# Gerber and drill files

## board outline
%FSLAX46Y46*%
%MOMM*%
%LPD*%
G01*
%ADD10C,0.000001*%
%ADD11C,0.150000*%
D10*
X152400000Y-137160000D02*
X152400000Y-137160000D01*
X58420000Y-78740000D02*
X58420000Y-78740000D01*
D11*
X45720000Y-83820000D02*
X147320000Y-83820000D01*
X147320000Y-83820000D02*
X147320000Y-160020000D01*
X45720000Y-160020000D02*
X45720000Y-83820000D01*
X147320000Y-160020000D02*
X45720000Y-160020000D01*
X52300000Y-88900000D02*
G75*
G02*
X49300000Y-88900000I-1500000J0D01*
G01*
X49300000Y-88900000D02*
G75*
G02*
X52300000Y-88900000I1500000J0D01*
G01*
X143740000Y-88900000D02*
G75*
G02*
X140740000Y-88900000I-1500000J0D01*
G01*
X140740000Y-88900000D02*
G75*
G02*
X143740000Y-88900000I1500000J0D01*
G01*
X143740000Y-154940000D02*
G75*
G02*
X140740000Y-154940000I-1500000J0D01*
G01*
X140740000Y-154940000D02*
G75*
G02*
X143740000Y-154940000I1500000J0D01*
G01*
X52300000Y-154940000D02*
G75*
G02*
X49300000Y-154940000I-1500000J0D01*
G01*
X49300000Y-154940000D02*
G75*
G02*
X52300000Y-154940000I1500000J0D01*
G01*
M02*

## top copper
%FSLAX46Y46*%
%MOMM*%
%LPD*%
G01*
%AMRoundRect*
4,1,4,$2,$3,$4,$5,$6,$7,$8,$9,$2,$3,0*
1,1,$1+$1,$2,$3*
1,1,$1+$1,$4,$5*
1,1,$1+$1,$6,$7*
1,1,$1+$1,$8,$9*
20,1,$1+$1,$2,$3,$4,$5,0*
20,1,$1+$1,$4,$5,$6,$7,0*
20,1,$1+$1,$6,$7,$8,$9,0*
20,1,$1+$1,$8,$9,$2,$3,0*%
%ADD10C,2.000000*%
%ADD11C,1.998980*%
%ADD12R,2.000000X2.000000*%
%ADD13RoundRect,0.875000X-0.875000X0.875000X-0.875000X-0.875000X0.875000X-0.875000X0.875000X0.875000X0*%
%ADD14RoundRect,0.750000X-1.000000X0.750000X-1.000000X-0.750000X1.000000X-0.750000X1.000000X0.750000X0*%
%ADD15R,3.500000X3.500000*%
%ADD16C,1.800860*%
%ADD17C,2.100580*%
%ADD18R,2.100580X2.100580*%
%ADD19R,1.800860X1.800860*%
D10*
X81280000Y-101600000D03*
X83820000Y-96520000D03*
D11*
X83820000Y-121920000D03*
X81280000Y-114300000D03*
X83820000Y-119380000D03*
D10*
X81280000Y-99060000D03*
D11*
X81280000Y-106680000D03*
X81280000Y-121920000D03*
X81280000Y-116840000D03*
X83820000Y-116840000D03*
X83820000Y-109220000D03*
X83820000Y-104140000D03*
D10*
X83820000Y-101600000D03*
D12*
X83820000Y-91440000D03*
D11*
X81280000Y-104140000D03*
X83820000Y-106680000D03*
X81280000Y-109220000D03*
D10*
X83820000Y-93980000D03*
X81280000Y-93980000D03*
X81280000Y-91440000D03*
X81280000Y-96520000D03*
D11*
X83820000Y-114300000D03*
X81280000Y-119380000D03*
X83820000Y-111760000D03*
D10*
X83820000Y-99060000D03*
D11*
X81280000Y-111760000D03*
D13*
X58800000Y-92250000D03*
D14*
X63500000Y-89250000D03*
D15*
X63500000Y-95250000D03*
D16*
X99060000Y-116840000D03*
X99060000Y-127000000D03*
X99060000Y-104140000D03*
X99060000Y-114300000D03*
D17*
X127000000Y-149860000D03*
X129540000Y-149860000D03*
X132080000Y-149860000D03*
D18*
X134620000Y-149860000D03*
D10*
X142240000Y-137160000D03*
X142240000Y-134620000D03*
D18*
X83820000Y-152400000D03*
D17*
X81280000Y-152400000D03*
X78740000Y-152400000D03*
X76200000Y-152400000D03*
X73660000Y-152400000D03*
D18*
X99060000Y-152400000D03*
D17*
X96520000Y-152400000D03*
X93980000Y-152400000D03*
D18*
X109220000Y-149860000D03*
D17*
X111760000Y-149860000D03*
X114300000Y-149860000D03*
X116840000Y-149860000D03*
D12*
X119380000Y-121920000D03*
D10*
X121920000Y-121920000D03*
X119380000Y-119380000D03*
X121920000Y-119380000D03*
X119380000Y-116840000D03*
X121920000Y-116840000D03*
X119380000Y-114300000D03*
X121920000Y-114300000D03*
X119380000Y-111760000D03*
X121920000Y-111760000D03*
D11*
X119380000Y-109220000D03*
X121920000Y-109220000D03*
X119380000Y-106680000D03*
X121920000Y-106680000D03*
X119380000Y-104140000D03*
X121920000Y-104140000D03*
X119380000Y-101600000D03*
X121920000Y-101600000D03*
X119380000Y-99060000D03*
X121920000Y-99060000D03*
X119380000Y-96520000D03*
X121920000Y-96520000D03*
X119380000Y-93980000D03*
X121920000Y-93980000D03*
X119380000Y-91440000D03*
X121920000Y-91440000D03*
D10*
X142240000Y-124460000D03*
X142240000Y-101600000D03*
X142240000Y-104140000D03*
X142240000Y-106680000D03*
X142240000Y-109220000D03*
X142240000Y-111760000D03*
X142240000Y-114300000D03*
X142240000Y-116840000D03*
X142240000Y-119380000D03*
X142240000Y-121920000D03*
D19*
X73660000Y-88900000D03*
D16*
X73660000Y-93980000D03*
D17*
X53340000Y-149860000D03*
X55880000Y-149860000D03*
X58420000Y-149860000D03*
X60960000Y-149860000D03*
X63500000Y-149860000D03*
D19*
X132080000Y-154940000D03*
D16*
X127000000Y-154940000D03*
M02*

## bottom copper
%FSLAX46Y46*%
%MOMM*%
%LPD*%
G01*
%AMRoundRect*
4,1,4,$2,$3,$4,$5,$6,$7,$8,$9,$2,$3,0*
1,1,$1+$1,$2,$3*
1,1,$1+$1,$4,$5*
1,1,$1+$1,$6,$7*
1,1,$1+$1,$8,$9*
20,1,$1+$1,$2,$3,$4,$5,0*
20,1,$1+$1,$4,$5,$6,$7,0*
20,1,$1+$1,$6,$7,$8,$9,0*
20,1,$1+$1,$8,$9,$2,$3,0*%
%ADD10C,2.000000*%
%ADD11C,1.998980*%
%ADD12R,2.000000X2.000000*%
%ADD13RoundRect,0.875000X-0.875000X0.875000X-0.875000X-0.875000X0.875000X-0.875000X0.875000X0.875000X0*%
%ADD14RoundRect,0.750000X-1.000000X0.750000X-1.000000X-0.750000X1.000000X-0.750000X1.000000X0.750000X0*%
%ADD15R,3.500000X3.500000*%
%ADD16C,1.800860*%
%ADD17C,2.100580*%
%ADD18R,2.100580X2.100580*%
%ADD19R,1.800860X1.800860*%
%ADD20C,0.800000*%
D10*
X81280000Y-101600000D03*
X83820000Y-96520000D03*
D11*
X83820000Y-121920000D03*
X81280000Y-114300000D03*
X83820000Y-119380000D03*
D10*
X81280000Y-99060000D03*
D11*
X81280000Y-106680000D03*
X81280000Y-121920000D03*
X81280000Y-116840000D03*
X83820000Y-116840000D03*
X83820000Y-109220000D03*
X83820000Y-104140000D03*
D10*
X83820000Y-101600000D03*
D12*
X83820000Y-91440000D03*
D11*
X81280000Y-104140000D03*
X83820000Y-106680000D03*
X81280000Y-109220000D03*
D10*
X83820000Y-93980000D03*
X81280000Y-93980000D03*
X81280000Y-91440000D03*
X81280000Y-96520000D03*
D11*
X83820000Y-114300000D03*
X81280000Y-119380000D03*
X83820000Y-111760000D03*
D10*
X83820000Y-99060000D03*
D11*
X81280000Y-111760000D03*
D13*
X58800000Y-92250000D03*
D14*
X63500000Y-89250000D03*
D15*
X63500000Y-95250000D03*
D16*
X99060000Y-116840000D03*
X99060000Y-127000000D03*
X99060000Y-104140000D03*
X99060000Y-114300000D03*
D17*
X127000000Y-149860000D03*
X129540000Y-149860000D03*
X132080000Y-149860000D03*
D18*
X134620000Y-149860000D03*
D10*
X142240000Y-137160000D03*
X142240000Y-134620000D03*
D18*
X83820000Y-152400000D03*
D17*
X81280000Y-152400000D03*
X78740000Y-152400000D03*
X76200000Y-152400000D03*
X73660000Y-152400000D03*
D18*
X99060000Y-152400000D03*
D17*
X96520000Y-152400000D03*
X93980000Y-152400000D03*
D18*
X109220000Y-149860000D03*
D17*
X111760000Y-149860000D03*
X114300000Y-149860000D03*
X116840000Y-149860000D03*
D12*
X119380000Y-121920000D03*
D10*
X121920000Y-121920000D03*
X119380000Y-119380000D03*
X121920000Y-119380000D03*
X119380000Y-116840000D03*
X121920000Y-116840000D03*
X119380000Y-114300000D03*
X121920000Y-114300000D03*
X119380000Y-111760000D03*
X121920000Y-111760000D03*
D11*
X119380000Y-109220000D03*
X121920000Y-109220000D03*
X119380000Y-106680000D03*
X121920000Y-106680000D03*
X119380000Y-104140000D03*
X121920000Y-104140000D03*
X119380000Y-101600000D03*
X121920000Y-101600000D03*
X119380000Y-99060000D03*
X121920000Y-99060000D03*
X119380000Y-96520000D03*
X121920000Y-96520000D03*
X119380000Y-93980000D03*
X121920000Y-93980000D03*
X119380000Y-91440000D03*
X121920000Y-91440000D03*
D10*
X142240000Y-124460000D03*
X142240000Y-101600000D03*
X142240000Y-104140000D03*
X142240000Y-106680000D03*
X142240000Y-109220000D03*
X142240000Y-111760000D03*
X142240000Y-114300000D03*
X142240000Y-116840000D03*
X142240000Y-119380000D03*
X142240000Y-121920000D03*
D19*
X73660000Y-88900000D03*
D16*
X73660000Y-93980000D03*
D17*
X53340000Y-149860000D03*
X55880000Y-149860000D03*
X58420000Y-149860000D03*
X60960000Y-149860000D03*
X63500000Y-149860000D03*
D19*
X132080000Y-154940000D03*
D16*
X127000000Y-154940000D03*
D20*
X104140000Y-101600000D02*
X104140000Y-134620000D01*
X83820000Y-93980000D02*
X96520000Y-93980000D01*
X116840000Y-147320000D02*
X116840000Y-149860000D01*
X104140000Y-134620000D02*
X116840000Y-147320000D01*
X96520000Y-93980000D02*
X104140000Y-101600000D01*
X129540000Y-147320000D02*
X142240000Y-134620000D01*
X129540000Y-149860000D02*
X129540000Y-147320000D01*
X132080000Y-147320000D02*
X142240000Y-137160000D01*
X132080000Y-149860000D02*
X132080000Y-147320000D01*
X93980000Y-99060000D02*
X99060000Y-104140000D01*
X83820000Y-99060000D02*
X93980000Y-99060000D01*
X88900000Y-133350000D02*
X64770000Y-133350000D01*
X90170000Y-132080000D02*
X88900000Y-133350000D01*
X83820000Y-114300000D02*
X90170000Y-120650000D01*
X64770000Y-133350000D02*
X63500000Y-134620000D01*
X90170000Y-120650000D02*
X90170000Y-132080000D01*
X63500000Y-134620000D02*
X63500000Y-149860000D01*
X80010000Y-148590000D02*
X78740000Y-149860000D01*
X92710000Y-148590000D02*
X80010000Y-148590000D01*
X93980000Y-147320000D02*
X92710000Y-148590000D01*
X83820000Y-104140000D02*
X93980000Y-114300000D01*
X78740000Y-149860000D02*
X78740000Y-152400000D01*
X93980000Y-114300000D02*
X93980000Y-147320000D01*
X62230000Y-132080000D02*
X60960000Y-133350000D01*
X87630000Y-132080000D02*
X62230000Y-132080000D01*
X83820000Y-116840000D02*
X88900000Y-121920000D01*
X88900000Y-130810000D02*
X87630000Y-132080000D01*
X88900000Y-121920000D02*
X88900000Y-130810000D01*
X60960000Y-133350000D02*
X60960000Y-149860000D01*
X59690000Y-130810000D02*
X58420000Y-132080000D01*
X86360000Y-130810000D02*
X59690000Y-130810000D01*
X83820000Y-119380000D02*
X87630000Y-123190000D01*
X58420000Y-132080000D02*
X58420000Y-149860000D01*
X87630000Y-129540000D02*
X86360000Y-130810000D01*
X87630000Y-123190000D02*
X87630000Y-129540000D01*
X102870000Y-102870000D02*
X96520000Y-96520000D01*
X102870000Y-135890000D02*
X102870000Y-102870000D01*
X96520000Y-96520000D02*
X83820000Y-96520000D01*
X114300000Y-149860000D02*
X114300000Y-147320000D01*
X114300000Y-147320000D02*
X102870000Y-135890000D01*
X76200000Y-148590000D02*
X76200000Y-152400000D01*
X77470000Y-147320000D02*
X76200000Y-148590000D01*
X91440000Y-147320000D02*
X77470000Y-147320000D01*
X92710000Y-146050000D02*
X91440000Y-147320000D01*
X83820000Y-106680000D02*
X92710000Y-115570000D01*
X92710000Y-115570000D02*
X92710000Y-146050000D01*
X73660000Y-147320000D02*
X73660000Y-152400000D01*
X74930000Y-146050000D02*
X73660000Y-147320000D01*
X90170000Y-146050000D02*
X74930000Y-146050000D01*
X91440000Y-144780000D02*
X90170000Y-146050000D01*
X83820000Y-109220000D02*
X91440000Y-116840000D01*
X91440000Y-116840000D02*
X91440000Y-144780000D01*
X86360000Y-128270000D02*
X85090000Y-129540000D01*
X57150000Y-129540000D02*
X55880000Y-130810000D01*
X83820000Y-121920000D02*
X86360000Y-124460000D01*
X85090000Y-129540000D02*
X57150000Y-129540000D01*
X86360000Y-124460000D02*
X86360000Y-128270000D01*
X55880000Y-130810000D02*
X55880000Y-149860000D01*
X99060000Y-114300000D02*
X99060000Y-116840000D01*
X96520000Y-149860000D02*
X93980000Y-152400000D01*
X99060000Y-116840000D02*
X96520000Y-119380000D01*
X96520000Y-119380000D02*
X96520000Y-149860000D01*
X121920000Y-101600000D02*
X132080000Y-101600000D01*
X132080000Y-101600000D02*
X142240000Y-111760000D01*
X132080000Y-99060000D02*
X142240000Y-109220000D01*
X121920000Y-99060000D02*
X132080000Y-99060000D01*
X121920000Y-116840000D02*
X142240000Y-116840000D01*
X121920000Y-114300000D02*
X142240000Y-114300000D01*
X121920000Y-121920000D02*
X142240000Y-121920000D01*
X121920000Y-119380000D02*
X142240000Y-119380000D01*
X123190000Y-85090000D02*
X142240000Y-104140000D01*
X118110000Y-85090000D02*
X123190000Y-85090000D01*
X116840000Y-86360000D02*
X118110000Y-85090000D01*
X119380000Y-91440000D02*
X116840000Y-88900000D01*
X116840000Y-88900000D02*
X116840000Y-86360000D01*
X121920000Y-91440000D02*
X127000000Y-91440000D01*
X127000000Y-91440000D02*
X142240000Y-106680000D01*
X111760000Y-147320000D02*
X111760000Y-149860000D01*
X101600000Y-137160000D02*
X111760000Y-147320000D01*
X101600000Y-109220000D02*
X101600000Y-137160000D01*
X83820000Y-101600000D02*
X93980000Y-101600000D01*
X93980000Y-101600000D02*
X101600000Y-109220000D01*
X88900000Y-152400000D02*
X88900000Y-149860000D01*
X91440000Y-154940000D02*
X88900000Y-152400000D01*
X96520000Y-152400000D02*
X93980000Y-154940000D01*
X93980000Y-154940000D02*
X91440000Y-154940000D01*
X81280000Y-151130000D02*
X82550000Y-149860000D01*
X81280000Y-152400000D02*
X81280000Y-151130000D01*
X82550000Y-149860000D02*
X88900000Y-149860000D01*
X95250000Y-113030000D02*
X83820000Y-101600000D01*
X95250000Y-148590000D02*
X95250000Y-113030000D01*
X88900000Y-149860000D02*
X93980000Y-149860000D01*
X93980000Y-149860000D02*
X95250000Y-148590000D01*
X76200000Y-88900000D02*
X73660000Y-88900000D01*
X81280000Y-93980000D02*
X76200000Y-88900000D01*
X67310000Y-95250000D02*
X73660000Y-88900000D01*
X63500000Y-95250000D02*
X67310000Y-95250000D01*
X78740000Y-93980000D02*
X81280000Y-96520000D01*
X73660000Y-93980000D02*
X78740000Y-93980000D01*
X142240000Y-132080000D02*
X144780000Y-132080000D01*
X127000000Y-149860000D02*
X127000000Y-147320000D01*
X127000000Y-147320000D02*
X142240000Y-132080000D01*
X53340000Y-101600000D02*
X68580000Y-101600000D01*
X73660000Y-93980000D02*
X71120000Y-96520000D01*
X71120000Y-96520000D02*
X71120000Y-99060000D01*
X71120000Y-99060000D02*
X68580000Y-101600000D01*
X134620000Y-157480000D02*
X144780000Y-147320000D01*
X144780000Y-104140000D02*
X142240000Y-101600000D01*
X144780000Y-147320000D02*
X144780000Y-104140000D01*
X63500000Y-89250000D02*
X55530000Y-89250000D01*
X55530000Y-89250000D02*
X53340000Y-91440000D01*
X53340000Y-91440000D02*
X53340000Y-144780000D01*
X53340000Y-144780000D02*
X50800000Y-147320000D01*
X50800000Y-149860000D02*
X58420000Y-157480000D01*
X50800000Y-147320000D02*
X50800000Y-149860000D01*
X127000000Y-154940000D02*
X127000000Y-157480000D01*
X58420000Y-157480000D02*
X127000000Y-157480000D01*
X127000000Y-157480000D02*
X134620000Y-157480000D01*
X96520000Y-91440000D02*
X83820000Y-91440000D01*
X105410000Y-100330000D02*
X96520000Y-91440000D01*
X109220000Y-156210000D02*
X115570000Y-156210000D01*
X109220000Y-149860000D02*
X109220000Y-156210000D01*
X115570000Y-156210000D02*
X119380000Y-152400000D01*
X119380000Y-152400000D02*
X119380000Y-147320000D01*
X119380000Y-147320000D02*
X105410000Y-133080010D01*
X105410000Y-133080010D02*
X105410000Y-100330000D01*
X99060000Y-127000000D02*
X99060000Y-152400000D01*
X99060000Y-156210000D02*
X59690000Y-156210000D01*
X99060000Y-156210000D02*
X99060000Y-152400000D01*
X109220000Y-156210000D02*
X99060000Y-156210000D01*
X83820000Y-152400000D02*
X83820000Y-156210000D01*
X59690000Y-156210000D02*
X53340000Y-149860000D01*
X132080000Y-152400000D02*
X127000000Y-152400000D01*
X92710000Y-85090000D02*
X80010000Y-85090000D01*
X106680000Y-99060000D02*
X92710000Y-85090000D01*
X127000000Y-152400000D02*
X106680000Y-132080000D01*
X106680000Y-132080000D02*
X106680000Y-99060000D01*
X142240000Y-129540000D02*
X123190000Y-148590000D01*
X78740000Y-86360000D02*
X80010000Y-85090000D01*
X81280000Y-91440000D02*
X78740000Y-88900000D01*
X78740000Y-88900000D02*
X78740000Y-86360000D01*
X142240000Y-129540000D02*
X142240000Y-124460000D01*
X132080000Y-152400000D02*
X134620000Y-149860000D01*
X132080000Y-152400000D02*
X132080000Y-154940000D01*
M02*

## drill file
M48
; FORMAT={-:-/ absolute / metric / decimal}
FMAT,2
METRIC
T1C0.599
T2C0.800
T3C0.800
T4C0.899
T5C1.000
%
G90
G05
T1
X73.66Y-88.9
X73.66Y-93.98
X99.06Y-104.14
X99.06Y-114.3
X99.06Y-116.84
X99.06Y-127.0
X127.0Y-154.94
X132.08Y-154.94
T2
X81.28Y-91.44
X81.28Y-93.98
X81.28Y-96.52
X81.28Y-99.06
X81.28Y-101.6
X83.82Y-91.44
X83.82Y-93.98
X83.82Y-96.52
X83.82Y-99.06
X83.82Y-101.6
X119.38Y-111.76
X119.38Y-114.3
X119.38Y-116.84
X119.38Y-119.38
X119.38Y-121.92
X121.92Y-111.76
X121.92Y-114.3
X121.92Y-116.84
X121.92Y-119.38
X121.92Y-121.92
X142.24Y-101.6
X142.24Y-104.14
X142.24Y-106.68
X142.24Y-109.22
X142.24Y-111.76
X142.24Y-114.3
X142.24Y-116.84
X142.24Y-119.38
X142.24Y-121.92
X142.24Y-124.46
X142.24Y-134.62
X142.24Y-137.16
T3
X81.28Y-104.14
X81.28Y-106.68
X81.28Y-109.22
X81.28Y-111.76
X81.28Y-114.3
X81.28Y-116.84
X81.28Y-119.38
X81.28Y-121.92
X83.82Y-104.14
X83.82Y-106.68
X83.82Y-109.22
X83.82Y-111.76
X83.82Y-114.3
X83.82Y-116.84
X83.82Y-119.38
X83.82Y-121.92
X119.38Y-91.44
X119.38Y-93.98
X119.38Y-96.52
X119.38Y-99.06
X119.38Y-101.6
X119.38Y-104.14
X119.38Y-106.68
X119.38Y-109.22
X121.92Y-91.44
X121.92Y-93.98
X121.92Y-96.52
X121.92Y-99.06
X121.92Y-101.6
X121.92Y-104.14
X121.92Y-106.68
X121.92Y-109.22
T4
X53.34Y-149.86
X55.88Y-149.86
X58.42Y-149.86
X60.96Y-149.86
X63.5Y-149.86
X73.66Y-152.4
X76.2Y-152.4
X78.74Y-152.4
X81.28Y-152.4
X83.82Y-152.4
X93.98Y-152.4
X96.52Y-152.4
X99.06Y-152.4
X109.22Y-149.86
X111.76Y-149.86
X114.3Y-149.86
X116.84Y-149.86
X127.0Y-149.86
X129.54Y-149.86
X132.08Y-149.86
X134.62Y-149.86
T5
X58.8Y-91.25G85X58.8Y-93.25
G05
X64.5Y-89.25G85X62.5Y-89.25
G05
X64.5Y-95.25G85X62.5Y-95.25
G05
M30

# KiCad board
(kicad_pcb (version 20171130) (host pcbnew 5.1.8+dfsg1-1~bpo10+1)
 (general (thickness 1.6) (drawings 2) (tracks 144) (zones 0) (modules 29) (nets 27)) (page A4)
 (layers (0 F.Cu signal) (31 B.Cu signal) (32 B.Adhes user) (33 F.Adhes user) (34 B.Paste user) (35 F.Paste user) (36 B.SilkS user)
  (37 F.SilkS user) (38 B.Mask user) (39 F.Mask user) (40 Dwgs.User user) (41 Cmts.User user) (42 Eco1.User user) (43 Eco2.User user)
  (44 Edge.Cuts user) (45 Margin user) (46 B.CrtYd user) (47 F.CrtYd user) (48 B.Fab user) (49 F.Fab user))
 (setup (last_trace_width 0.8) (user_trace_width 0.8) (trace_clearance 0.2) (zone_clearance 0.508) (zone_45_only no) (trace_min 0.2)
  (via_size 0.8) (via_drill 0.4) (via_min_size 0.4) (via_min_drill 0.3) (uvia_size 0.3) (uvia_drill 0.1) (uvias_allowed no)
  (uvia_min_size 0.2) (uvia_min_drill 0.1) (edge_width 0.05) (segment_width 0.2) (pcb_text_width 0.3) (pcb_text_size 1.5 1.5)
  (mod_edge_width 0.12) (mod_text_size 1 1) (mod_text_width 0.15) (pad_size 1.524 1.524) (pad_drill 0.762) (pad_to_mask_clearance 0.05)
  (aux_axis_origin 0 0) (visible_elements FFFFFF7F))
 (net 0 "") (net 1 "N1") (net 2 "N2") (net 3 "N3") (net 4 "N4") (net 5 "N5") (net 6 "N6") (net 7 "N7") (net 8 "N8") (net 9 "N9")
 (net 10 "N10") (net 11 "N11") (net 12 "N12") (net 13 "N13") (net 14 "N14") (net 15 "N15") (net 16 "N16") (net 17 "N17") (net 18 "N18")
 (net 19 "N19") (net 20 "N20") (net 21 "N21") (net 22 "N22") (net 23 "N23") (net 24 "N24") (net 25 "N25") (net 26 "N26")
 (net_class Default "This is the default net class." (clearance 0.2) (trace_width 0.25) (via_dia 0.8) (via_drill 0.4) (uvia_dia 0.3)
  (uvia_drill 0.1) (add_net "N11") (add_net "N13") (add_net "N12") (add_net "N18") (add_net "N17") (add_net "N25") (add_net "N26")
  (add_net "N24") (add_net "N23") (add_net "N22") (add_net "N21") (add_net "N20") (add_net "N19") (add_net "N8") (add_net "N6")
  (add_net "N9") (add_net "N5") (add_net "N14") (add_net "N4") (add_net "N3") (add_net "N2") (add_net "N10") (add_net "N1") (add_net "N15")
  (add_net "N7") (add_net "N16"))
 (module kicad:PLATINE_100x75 (layer F.Cu) (at 96.52 121.92)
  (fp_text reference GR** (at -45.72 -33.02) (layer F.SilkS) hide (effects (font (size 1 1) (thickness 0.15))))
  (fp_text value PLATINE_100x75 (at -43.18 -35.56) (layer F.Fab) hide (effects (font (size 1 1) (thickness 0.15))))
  (fp_line (start -50.8 -38.1) (end 50.8 -38.1) (layer Edge.Cuts) (width 0.15))
  (fp_line (start 50.8 -38.1) (end 50.8 38.1) (layer Edge.Cuts) (width 0.15))
  (fp_line (start -50.8 38.1) (end -50.8 -38.1) (layer Edge.Cuts) (width 0.15))
  (fp_line (start 50.8 38.1) (end -50.8 38.1) (layer Edge.Cuts) (width 0.15)))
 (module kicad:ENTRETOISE (layer F.Cu) (at 50.8 88.9)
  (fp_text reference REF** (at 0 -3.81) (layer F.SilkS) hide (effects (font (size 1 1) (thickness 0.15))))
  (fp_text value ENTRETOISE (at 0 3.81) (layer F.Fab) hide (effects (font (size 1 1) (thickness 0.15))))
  (fp_circle (center 0 0) (end 1.5 0) (layer Edge.Cuts) (width 0.15)))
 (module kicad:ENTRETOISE (layer F.Cu) (at 142.24 88.9)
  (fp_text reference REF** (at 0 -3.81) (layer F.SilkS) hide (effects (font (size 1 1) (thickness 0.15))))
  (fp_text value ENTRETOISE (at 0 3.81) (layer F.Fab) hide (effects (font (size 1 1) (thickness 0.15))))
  (fp_circle (center 0 0) (end 1.5 0) (layer Edge.Cuts) (width 0.15)))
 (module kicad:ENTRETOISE (layer F.Cu) (at 142.24 154.94)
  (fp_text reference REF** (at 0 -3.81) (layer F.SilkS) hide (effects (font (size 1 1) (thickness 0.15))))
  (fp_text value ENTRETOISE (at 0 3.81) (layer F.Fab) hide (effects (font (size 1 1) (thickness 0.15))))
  (fp_circle (center 0 0) (end 1.5 0) (layer Edge.Cuts) (width 0.15)))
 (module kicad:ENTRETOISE (layer F.Cu) (at 50.8 154.94)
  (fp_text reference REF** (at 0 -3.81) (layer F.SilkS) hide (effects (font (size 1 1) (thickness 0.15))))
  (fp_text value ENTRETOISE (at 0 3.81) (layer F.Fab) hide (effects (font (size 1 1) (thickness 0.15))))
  (fp_circle (center 0 0) (end 1.5 0) (layer Edge.Cuts) (width 0.15)))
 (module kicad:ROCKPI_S (layer F.Cu) (at 101.6 106.68)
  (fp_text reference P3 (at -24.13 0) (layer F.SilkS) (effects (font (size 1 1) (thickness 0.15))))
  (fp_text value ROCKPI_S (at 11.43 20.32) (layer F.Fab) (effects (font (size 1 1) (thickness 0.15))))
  (pad 10 thru_hole circle (at -20.32 -5.08 270) (size 2 2) (drill 0.8) (layers *.Cu *.Mask F.SilkS))
  (pad 5 thru_hole circle (at -17.78 -10.16 270) (size 2 2) (drill 0.8) (layers *.Cu *.Mask F.SilkS) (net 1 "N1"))
  (pad 25 thru_hole circle (at -17.78 15.24 270) (size 1.99898 1.99898) (drill 0.8001) (layers *.Cu *.Mask F.SilkS) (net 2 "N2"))
  (pad 20 thru_hole circle (at -20.32 7.62 270) (size 1.99898 1.99898) (drill 0.8001) (layers *.Cu *.Mask F.SilkS))
  (pad 23 thru_hole circle (at -17.78 12.7 270) (size 1.99898 1.99898) (drill 0.8001) (layers *.Cu *.Mask F.SilkS) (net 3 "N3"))
  (pad 8 thru_hole circle (at -20.32 -7.62 270) (size 2 2) (drill 0.8) (layers *.Cu *.Mask F.SilkS))
  (pad 14 thru_hole circle (at -20.32 0 270) (size 1.99898 1.99898) (drill 0.8001) (layers *.Cu *.Mask F.SilkS))
  (pad 26 thru_hole circle (at -20.32 15.24 270) (size 1.99898 1.99898) (drill 0.8001) (layers *.Cu *.Mask F.SilkS))
  (pad 22 thru_hole circle (at -20.32 10.16 270) (size 1.99898 1.99898) (drill 0.8001) (layers *.Cu *.Mask F.SilkS))
  (pad 21 thru_hole circle (at -17.78 10.16 270) (size 1.99898 1.99898) (drill 0.8001) (layers *.Cu *.Mask F.SilkS) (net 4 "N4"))
  (pad 15 thru_hole circle (at -17.78 2.54 270) (size 1.99898 1.99898) (drill 0.8001) (layers *.Cu *.Mask F.SilkS) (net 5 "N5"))
  (pad 11 thru_hole circle (at -17.78 -2.54 270) (size 1.99898 1.99898) (drill 0.8001) (layers *.Cu *.Mask F.SilkS) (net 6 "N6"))
  (pad 9 thru_hole circle (at -17.78 -5.08 270) (size 2 2) (drill 0.8) (layers *.Cu *.Mask F.SilkS) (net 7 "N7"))
  (pad 1 thru_hole rect (at -17.78 -15.24 270) (size 2 2) (drill 0.8) (layers *.Cu *.Mask F.SilkS) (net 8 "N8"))
  (pad 12 thru_hole circle (at -20.32 -2.54 270) (size 1.99898 1.99898) (drill 0.8001) (layers *.Cu *.Mask F.SilkS))
  (pad 13 thru_hole circle (at -17.78 0 270) (size 1.99898 1.99898) (drill 0.8001) (layers *.Cu *.Mask F.SilkS) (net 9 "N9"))
  (pad 16 thru_hole circle (at -20.32 2.54 270) (size 1.99898 1.99898) (drill 0.8001) (layers *.Cu *.Mask F.SilkS))
  (pad 3 thru_hole circle (at -17.78 -12.7 270) (size 2 2) (drill 0.8) (layers *.Cu *.Mask F.SilkS) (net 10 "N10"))
  (pad 4 thru_hole circle (at -20.32 -12.7 270) (size 2 2) (drill 0.8) (layers *.Cu *.Mask F.SilkS) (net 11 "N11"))
  (pad 2 thru_hole circle (at -20.32 -15.24 270) (size 2 2) (drill 0.8) (layers *.Cu *.Mask F.SilkS) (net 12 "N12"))
  (pad 6 thru_hole circle (at -20.32 -10.16 270) (size 2 2) (drill 0.8) (layers *.Cu *.Mask F.SilkS) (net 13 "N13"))
  (pad 19 thru_hole circle (at -17.78 7.62 270) (size 1.99898 1.99898) (drill 0.8001) (layers *.Cu *.Mask F.SilkS) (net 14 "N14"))
  (pad 24 thru_hole circle (at -20.32 12.7 270) (size 1.99898 1.99898) (drill 0.8001) (layers *.Cu *.Mask F.SilkS))
  (pad 17 thru_hole circle (at -17.78 5.08) (size 1.99898 1.99898) (drill 0.8001) (layers *.Cu *.Mask F.SilkS))
  (pad 7 thru_hole circle (at -17.78 -7.62 270) (size 2 2) (drill 0.8) (layers *.Cu *.Mask F.SilkS) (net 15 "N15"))
  (pad 18 thru_hole circle (at -20.32 5.08 270) (size 1.99898 1.99898) (drill 0.8001) (layers *.Cu *.Mask F.SilkS)))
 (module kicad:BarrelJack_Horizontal (layer F.Cu) (at 63.5 95.25 270)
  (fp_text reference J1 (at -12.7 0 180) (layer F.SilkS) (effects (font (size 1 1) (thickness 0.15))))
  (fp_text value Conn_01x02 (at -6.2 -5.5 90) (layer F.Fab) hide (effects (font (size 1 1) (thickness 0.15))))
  (pad 3 thru_hole roundrect (at -3 4.7 270) (size 3.5 3.5) (drill oval 3 1) (layers *.Cu *.Mask) (roundrect_rratio 0.25))
  (pad 2 thru_hole roundrect (at -6 0 270) (size 3 3.5) (drill oval 1 3) (layers *.Cu *.Mask) (roundrect_rratio 0.25) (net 13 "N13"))
  (pad 1 thru_hole rect (at 0 0 270) (size 3.5 3.5) (drill oval 1 3) (layers *.Cu *.Mask) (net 11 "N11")))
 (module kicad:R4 (layer F.Cu) (at 99.06 121.92 270) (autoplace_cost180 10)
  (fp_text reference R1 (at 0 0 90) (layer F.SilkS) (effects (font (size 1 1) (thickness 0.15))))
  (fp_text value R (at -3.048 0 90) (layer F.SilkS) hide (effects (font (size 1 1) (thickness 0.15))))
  (pad 1 thru_hole circle (at -5.08 0 270) (size 1.80086 1.80086) (drill 0.59944) (layers *.Cu *.Mask F.SilkS) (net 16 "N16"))
  (pad 2 thru_hole circle (at 5.08 0 270) (size 1.80086 1.80086) (drill 0.59944) (layers *.Cu *.Mask F.SilkS) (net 8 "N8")))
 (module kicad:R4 (layer F.Cu) (at 99.06 109.22 270) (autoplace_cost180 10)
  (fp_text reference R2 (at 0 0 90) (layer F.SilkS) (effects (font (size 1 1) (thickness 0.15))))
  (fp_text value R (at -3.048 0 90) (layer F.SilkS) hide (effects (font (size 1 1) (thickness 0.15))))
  (pad 1 thru_hole circle (at -5.08 0 270) (size 1.80086 1.80086) (drill 0.59944) (layers *.Cu *.Mask F.SilkS) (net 15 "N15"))
  (pad 2 thru_hole circle (at 5.08 0 270) (size 1.80086 1.80086) (drill 0.59944) (layers *.Cu *.Mask F.SilkS) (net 16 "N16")))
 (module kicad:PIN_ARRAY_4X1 (layer F.Cu) (at 130.81 149.86 180)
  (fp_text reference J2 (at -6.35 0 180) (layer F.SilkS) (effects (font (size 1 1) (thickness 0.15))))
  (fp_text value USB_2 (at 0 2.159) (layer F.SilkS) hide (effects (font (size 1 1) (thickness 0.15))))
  (pad 4 thru_hole circle (at 3.81 0 180) (size 2.10058 2.10058) (drill 0.89916) (layers *.Cu *.Mask F.SilkS) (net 13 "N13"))
  (pad 3 thru_hole circle (at 1.27 0 180) (size 2.10058 2.10058) (drill 0.89916) (layers *.Cu *.Mask F.SilkS) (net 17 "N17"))
  (pad 2 thru_hole circle (at -1.27 0 180) (size 2.10058 2.10058) (drill 0.89916) (layers *.Cu *.Mask F.SilkS) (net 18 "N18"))
  (pad 1 thru_hole rect (at -3.81 0 180) (size 2.10058 2.10058) (drill 0.89916) (layers *.Cu *.Mask F.SilkS) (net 12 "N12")))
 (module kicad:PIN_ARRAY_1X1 (layer F.Cu) (at 142.24 137.16)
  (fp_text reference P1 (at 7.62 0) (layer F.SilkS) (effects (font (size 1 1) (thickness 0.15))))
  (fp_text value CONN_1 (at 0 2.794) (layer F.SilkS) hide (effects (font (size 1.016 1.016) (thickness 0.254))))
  (pad 1 thru_hole circle (at 0 0) (size 2 2) (drill 0.8) (layers *.Cu *.Mask F.SilkS) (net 18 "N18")))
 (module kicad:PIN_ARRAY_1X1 (layer F.Cu) (at 142.24 134.62)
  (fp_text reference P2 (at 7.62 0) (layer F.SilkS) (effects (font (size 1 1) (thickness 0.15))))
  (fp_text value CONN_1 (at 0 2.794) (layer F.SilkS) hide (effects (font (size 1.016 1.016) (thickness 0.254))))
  (pad 1 thru_hole circle (at 0 0) (size 2 2) (drill 0.8) (layers *.Cu *.Mask F.SilkS) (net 17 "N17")))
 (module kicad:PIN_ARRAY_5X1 (layer F.Cu) (at 78.74 152.4 180)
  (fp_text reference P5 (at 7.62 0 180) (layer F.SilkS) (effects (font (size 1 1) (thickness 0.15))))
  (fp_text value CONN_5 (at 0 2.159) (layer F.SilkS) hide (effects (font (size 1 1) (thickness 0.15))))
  (pad 1 thru_hole rect (at -5.08 0 180) (size 2.10058 2.10058) (drill 0.89916) (layers *.Cu *.Mask F.SilkS) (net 8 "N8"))
  (pad 2 thru_hole circle (at -2.54 0 180) (size 2.10058 2.10058) (drill 0.89916) (layers *.Cu *.Mask F.SilkS) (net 7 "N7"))
  (pad 3 thru_hole circle (at 0 0 180) (size 2.10058 2.10058) (drill 0.89916) (layers *.Cu *.Mask F.SilkS) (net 6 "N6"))
  (pad 4 thru_hole circle (at 2.54 0 180) (size 2.10058 2.10058) (drill 0.89916) (layers *.Cu *.Mask F.SilkS) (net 9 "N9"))
  (pad 5 thru_hole circle (at 5.08 0 180) (size 2.10058 2.10058) (drill 0.89916) (layers *.Cu *.Mask F.SilkS) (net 5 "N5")))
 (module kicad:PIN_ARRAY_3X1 (layer F.Cu) (at 96.52 152.4 180)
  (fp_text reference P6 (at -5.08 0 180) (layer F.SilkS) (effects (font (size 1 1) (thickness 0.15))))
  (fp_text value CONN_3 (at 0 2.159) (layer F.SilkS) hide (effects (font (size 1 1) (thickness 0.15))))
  (pad 1 thru_hole rect (at -2.54 0 180) (size 2.10058 2.10058) (drill 0.89916) (layers *.Cu *.Mask F.SilkS) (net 8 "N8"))
  (pad 2 thru_hole circle (at 0 0 180) (size 2.10058 2.10058) (drill 0.89916) (layers *.Cu *.Mask F.SilkS) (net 7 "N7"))
  (pad 3 thru_hole circle (at 2.54 0 180) (size 2.10058 2.10058) (drill 0.89916) (layers *.Cu *.Mask F.SilkS) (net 16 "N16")))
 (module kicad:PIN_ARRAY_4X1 (layer F.Cu) (at 113.03 149.86)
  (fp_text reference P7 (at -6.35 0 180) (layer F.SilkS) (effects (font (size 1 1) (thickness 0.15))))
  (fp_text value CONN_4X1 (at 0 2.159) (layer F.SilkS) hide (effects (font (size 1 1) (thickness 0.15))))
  (pad 1 thru_hole rect (at -3.81 0) (size 2.10058 2.10058) (drill 0.89916) (layers *.Cu *.Mask F.SilkS) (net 8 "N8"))
  (pad 2 thru_hole circle (at -1.27 0) (size 2.10058 2.10058) (drill 0.89916) (layers *.Cu *.Mask F.SilkS) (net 7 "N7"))
  (pad 3 thru_hole circle (at 1.27 0) (size 2.10058 2.10058) (drill 0.89916) (layers *.Cu *.Mask F.SilkS) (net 1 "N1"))
  (pad 4 thru_hole circle (at 3.81 0) (size 2.10058 2.10058) (drill 0.89916) (layers *.Cu *.Mask F.SilkS) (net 10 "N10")))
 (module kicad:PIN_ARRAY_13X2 (layer F.Cu) (at 120.65 106.68 90)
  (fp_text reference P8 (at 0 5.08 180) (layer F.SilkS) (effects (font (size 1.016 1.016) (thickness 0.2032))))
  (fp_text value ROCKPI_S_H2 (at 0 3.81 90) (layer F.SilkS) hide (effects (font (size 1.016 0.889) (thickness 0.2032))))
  (pad 1 thru_hole rect (at -15.24 -1.27 90) (size 2 2) (drill 0.8) (layers *.Cu *.Mask F.SilkS))
  (pad 2 thru_hole circle (at -15.24 1.27 90) (size 2 2) (drill 0.8) (layers *.Cu *.Mask F.SilkS) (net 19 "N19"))
  (pad 3 thru_hole circle (at -12.7 -1.27 90) (size 2 2) (drill 0.8) (layers *.Cu *.Mask F.SilkS))
  (pad 4 thru_hole circle (at -12.7 1.27 90) (size 2 2) (drill 0.8) (layers *.Cu *.Mask F.SilkS) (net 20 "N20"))
  (pad 5 thru_hole circle (at -10.16 -1.27 90) (size 2 2) (drill 0.8) (layers *.Cu *.Mask F.SilkS))
  (pad 6 thru_hole circle (at -10.16 1.27 90) (size 2 2) (drill 0.8) (layers *.Cu *.Mask F.SilkS) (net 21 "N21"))
  (pad 7 thru_hole circle (at -7.62 -1.27 90) (size 2 2) (drill 0.8) (layers *.Cu *.Mask F.SilkS))
  (pad 8 thru_hole circle (at -7.62 1.27 90) (size 2 2) (drill 0.8) (layers *.Cu *.Mask F.SilkS) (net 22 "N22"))
  (pad 9 thru_hole circle (at -5.08 -1.27 90) (size 2 2) (drill 0.8) (layers *.Cu *.Mask F.SilkS))
  (pad 10 thru_hole circle (at -5.08 1.27 90) (size 2 2) (drill 0.8) (layers *.Cu *.Mask F.SilkS))
  (pad 11 thru_hole circle (at -2.54 -1.27 90) (size 1.99898 1.99898) (drill 0.8001) (layers *.Cu *.Mask F.SilkS))
  (pad 12 thru_hole circle (at -2.54 1.27 90) (size 1.99898 1.99898) (drill 0.8001) (layers *.Cu *.Mask F.SilkS))
  (pad 13 thru_hole circle (at 0 -1.27 90) (size 1.99898 1.99898) (drill 0.8001) (layers *.Cu *.Mask F.SilkS))
  (pad 14 thru_hole circle (at 0 1.27 90) (size 1.99898 1.99898) (drill 0.8001) (layers *.Cu *.Mask F.SilkS))
  (pad 15 thru_hole circle (at 2.54 -1.27 90) (size 1.99898 1.99898) (drill 0.8001) (layers *.Cu *.Mask F.SilkS))
  (pad 16 thru_hole circle (at 2.54 1.27 90) (size 1.99898 1.99898) (drill 0.8001) (layers *.Cu *.Mask F.SilkS))
  (pad 17 thru_hole circle (at 5.08 -1.27 90) (size 1.99898 1.99898) (drill 0.8001) (layers *.Cu *.Mask F.SilkS))
  (pad 18 thru_hole circle (at 5.08 1.27 90) (size 1.99898 1.99898) (drill 0.8001) (layers *.Cu *.Mask F.SilkS) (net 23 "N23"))
  (pad 19 thru_hole circle (at 7.62 -1.27 90) (size 1.99898 1.99898) (drill 0.8001) (layers *.Cu *.Mask F.SilkS))
  (pad 20 thru_hole circle (at 7.62 1.27 90) (size 1.99898 1.99898) (drill 0.8001) (layers *.Cu *.Mask F.SilkS) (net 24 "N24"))
  (pad 21 thru_hole circle (at 10.16 -1.27 90) (size 1.99898 1.99898) (drill 0.8001) (layers *.Cu *.Mask F.SilkS))
  (pad 22 thru_hole circle (at 10.16 1.27 90) (size 1.99898 1.99898) (drill 0.8001) (layers *.Cu *.Mask F.SilkS))
  (pad 23 thru_hole circle (at 12.7 -1.27 90) (size 1.99898 1.99898) (drill 0.8001) (layers *.Cu *.Mask F.SilkS))
  (pad 24 thru_hole circle (at 12.7 1.27 90) (size 1.99898 1.99898) (drill 0.8001) (layers *.Cu *.Mask F.SilkS))
  (pad 25 thru_hole circle (at 15.24 -1.27 90) (size 1.99898 1.99898) (drill 0.8001) (layers *.Cu *.Mask F.SilkS) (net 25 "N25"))
  (pad 26 thru_hole circle (at 15.24 1.27 90) (size 1.99898 1.99898) (drill 0.8001) (layers *.Cu *.Mask F.SilkS) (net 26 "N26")))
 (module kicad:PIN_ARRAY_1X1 (layer F.Cu) (at 142.24 124.46 90)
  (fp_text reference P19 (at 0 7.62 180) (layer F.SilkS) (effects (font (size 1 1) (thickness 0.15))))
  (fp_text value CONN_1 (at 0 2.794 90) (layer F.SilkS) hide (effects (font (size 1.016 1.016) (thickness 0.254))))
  (pad 1 thru_hole circle (at 0 0 90) (size 2 2) (drill 0.8) (layers *.Cu *.Mask F.SilkS) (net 12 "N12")))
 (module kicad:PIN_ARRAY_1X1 (layer F.Cu) (at 142.24 101.6 90)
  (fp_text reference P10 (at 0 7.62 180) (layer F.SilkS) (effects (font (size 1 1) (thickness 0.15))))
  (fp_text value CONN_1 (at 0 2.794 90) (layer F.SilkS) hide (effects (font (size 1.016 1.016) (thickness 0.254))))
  (pad 1 thru_hole circle (at 0 0 90) (size 2 2) (drill 0.8) (layers *.Cu *.Mask F.SilkS) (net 13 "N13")))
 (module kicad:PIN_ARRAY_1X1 (layer F.Cu) (at 142.24 104.14 90)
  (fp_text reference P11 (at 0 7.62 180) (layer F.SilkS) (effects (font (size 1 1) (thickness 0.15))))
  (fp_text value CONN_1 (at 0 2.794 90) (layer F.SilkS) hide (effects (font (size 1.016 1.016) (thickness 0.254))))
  (pad 1 thru_hole circle (at 0 0 90) (size 2 2) (drill 0.8) (layers *.Cu *.Mask F.SilkS) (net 25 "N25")))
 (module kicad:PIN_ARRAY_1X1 (layer F.Cu) (at 142.24 106.68)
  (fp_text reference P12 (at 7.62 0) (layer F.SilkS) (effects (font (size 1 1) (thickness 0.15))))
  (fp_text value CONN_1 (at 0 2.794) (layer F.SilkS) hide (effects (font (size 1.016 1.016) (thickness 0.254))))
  (pad 1 thru_hole circle (at 0 0) (size 2 2) (drill 0.8) (layers *.Cu *.Mask F.SilkS) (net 26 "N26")))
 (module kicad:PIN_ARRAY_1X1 (layer F.Cu) (at 142.24 109.22)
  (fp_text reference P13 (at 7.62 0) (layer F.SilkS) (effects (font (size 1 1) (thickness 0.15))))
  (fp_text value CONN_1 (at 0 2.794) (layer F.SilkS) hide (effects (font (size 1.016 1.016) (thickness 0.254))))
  (pad 1 thru_hole circle (at 0 0) (size 2 2) (drill 0.8) (layers *.Cu *.Mask F.SilkS) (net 24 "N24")))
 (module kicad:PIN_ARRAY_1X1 (layer F.Cu) (at 142.24 111.76)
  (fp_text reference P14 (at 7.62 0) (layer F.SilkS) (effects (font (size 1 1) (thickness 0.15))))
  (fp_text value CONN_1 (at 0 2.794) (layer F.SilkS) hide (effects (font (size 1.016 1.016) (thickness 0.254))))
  (pad 1 thru_hole circle (at 0 0) (size 2 2) (drill 0.8) (layers *.Cu *.Mask F.SilkS) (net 23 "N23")))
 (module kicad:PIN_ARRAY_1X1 (layer F.Cu) (at 142.24 114.3)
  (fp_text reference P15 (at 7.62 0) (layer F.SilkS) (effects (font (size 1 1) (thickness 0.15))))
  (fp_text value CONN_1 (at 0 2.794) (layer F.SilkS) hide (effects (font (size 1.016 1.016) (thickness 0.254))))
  (pad 1 thru_hole circle (at 0 0) (size 2 2) (drill 0.8) (layers *.Cu *.Mask F.SilkS) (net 22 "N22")))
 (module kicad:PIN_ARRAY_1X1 (layer F.Cu) (at 142.24 116.84)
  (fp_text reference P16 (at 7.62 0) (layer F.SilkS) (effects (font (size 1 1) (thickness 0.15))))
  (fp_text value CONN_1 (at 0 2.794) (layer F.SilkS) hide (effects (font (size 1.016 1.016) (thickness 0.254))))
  (pad 1 thru_hole circle (at 0 0) (size 2 2) (drill 0.8) (layers *.Cu *.Mask F.SilkS) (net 21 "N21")))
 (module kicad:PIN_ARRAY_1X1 (layer F.Cu) (at 142.24 119.38)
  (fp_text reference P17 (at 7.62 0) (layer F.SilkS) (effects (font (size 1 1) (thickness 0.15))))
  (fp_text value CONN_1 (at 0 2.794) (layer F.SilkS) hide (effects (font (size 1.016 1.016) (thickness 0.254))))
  (pad 1 thru_hole circle (at 0 0) (size 2 2) (drill 0.8) (layers *.Cu *.Mask F.SilkS) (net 20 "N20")))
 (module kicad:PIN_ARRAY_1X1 (layer F.Cu) (at 142.24 121.92)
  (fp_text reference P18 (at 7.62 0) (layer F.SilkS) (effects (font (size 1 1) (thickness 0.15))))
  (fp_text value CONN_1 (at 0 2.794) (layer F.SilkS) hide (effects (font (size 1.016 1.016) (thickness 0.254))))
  (pad 1 thru_hole circle (at 0 0) (size 2 2) (drill 0.8) (layers *.Cu *.Mask F.SilkS) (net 19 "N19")))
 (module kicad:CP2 (layer F.Cu) (at 73.66 91.44 180)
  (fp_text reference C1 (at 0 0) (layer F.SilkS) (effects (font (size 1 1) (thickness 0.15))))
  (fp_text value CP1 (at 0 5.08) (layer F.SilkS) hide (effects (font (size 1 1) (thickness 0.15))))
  (pad 1 thru_hole rect (at 0 2.54 180) (size 1.80086 1.80086) (drill 0.59944) (layers *.Cu *.Mask F.SilkS) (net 11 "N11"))
  (pad 2 thru_hole circle (at 0 -2.54 180) (size 1.80086 1.80086) (drill 0.59944) (layers *.Cu *.Mask F.SilkS) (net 13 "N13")))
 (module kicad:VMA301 (layer F.Cu) (at 58.42 149.86)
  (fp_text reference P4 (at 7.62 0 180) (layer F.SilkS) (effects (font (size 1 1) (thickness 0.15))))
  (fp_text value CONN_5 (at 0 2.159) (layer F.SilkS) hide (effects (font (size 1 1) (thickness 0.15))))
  (pad 1 thru_hole circle (at -5.08 0) (size 2.10058 2.10058) (drill 0.89916) (layers *.Cu *.Mask F.SilkS) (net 8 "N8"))
  (pad 2 thru_hole circle (at -2.54 0) (size 2.10058 2.10058) (drill 0.89916) (layers *.Cu *.Mask F.SilkS) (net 2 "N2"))
  (pad 3 thru_hole circle (at 0 0) (size 2.10058 2.10058) (drill 0.89916) (layers *.Cu *.Mask F.SilkS) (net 3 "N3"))
  (pad 4 thru_hole circle (at 2.54 0) (size 2.10058 2.10058) (drill 0.89916) (layers *.Cu *.Mask F.SilkS) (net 4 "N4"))
  (pad 5 thru_hole circle (at 5.08 0) (size 2.10058 2.10058) (drill 0.89916) (layers *.Cu *.Mask F.SilkS) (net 14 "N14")))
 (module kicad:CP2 (layer F.Cu) (at 129.54 154.94 90)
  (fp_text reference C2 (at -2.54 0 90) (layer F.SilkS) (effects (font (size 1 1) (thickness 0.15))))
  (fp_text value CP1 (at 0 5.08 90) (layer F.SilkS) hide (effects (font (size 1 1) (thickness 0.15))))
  (pad 1 thru_hole rect (at 0 2.54 90) (size 1.80086 1.80086) (drill 0.59944) (layers *.Cu *.Mask F.SilkS) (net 12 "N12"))
  (pad 2 thru_hole circle (at 0 -2.54 90) (size 1.80086 1.80086) (drill 0.59944) (layers *.Cu *.Mask F.SilkS) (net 13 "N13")))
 (gr_line (start 152.4 137.16) (end 152.4 137.16) (layer Edge.Cuts) (width 0.000001))
 (gr_line (start 58.42 78.74) (end 58.42 78.74) (layer Edge.Cuts) (width 0.000001))
 (segment (start 104.14 101.6) (end 104.14 134.62) (width 0.8) (layer B.Cu) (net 10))
 (segment (start 83.82 93.98) (end 96.52 93.98) (width 0.8) (layer B.Cu) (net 10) (status 10))
 (segment (start 116.84 147.32) (end 116.84 149.86) (width 0.8) (layer B.Cu) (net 10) (status 20))
 (segment (start 104.14 134.62) (end 116.84 147.32) (width 0.8) (layer B.Cu) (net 10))
 (segment (start 96.52 93.98) (end 104.14 101.6) (width 0.8) (layer B.Cu) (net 10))
 (segment (start 129.54 147.32) (end 142.24 134.62) (width 0.8) (layer B.Cu) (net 17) (status 20))
 (segment (start 129.54 149.86) (end 129.54 147.32) (width 0.8) (layer B.Cu) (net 17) (status 10))
 (segment (start 132.08 147.32) (end 142.24 137.16) (width 0.8) (layer B.Cu) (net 18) (status 20))
 (segment (start 132.08 149.86) (end 132.08 147.32) (width 0.8) (layer B.Cu) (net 18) (status 10))
 (segment (start 93.98 99.06) (end 99.06 104.14) (width 0.8) (layer B.Cu) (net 15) (status 20))
 (segment (start 83.82 99.06) (end 93.98 99.06) (width 0.8) (layer B.Cu) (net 15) (status 10))
 (segment (start 88.9 133.35) (end 64.77 133.35) (width 0.8) (layer B.Cu) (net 14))
 (segment (start 90.17 132.08) (end 88.9 133.35) (width 0.8) (layer B.Cu) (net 14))
 (segment (start 83.82 114.3) (end 90.17 120.65) (width 0.8) (layer B.Cu) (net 14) (status 10))
 (segment (start 64.77 133.35) (end 63.5 134.62) (width 0.8) (layer B.Cu) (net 14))
 (segment (start 90.17 120.65) (end 90.17 132.08) (width 0.8) (layer B.Cu) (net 14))
 (segment (start 63.5 134.62) (end 63.5 149.86) (width 0.8) (layer B.Cu) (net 14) (status 20))
 (segment (start 80.01 148.59) (end 78.74 149.86) (width 0.8) (layer B.Cu) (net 6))
 (segment (start 92.71 148.59) (end 80.01 148.59) (width 0.8) (layer B.Cu) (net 6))
 (segment (start 93.98 147.32) (end 92.71 148.59) (width 0.8) (layer B.Cu) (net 6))
 (segment (start 83.82 104.14) (end 93.98 114.3) (width 0.8) (layer B.Cu) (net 6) (status 10))
 (segment (start 78.74 149.86) (end 78.74 152.4) (width 0.8) (layer B.Cu) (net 6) (status 20))
 (segment (start 93.98 114.3) (end 93.98 147.32) (width 0.8) (layer B.Cu) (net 6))
 (segment (start 62.23 132.08) (end 60.96 133.35) (width 0.8) (layer B.Cu) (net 4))
 (segment (start 87.63 132.08) (end 62.23 132.08) (width 0.8) (layer B.Cu) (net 4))
 (segment (start 83.82 116.84) (end 88.9 121.92) (width 0.8) (layer B.Cu) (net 4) (status 10))
 (segment (start 88.9 130.81) (end 87.63 132.08) (width 0.8) (layer B.Cu) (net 4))
 (segment (start 88.9 121.92) (end 88.9 130.81) (width 0.8) (layer B.Cu) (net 4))
 (segment (start 60.96 133.35) (end 60.96 149.86) (width 0.8) (layer B.Cu) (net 4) (status 20))
 (segment (start 59.69 130.81) (end 58.42 132.08) (width 0.8) (layer B.Cu) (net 3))
 (segment (start 86.36 130.81) (end 59.69 130.81) (width 0.8) (layer B.Cu) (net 3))
 (segment (start 83.82 119.38) (end 87.63 123.19) (width 0.8) (layer B.Cu) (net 3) (status 10))
 (segment (start 58.42 132.08) (end 58.42 149.86) (width 0.8) (layer B.Cu) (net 3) (status 20))
 (segment (start 87.63 129.54) (end 86.36 130.81) (width 0.8) (layer B.Cu) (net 3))
 (segment (start 87.63 123.19) (end 87.63 129.54) (width 0.8) (layer B.Cu) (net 3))
 (segment (start 102.87 102.87) (end 96.52 96.52) (width 0.8) (layer B.Cu) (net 1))
 (segment (start 102.87 135.89) (end 102.87 102.87) (width 0.8) (layer B.Cu) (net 1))
 (segment (start 96.52 96.52) (end 83.82 96.52) (width 0.8) (layer B.Cu) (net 1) (status 20))
 (segment (start 114.3 149.86) (end 114.3 147.32) (width 0.8) (layer B.Cu) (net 1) (status 10))
 (segment (start 114.3 147.32) (end 102.87 135.89) (width 0.8) (layer B.Cu) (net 1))
 (segment (start 76.2 148.59) (end 76.2 152.4) (width 0.8) (layer B.Cu) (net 9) (status 20))
 (segment (start 77.47 147.32) (end 76.2 148.59) (width 0.8) (layer B.Cu) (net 9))
 (segment (start 91.44 147.32) (end 77.47 147.32) (width 0.8) (layer B.Cu) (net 9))
 (segment (start 92.71 146.05) (end 91.44 147.32) (width 0.8) (layer B.Cu) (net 9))
 (segment (start 83.82 106.68) (end 92.71 115.57) (width 0.8) (layer B.Cu) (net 9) (status 10))
 (segment (start 92.71 115.57) (end 92.71 146.05) (width 0.8) (layer B.Cu) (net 9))
 (segment (start 73.66 147.32) (end 73.66 152.4) (width 0.8) (layer B.Cu) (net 5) (status 20))
 (segment (start 74.93 146.05) (end 73.66 147.32) (width 0.8) (layer B.Cu) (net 5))
 (segment (start 90.17 146.05) (end 74.93 146.05) (width 0.8) (layer B.Cu) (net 5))
 (segment (start 91.44 144.78) (end 90.17 146.05) (width 0.8) (layer B.Cu) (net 5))
 (segment (start 83.82 109.22) (end 91.44 116.84) (width 0.8) (layer B.Cu) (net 5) (status 10))
 (segment (start 91.44 116.84) (end 91.44 144.78) (width 0.8) (layer B.Cu) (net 5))
 (segment (start 86.36 128.27) (end 85.09 129.54) (width 0.8) (layer B.Cu) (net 2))
 (segment (start 57.15 129.54) (end 55.88 130.81) (width 0.8) (layer B.Cu) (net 2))
 (segment (start 83.82 121.92) (end 86.36 124.46) (width 0.8) (layer B.Cu) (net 2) (status 10))
 (segment (start 85.09 129.54) (end 57.15 129.54) (width 0.8) (layer B.Cu) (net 2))
 (segment (start 86.36 124.46) (end 86.36 128.27) (width 0.8) (layer B.Cu) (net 2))
 (segment (start 55.88 130.81) (end 55.88 149.86) (width 0.8) (layer B.Cu) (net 2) (status 20))
 (segment (start 99.06 114.3) (end 99.06 116.84) (width 0.8) (layer B.Cu) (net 16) (status 30))
 (segment (start 96.52 149.86) (end 93.98 152.4) (width 0.8) (layer B.Cu) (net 16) (status 20))
 (segment (start 99.06 116.84) (end 96.52 119.38) (width 0.8) (layer B.Cu) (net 16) (status 10))
 (segment (start 96.52 119.38) (end 96.52 149.86) (width 0.8) (layer B.Cu) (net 16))
 (segment (start 121.92 101.6) (end 132.08 101.6) (width 0.8) (layer B.Cu) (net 23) (status 10))
 (segment (start 132.08 101.6) (end 142.24 111.76) (width 0.8) (layer B.Cu) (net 23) (status 20))
 (segment (start 132.08 99.06) (end 142.24 109.22) (width 0.8) (layer B.Cu) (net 24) (status 20))
 (segment (start 121.92 99.06) (end 132.08 99.06) (width 0.8) (layer B.Cu) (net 24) (status 10))
 (segment (start 121.92 116.84) (end 142.24 116.84) (width 0.8) (layer B.Cu) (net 21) (status 30))
 (segment (start 121.92 114.3) (end 142.24 114.3) (width 0.8) (layer B.Cu) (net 22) (status 30))
 (segment (start 121.92 121.92) (end 142.24 121.92) (width 0.8) (layer B.Cu) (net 19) (status 30))
 (segment (start 121.92 119.38) (end 142.24 119.38) (width 0.8) (layer B.Cu) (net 20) (status 30))
 (segment (start 123.19 85.09) (end 142.24 104.14) (width 0.8) (layer B.Cu) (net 25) (status 20))
 (segment (start 118.11 85.09) (end 123.19 85.09) (width 0.8) (layer B.Cu) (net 25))
 (segment (start 116.84 86.36) (end 118.11 85.09) (width 0.8) (layer B.Cu) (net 25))
 (segment (start 119.38 91.44) (end 116.84 88.9) (width 0.8) (layer B.Cu) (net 25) (status 10))
 (segment (start 116.84 88.9) (end 116.84 86.36) (width 0.8) (layer B.Cu) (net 25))
 (segment (start 121.92 91.44) (end 127 91.44) (width 0.8) (layer B.Cu) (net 26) (status 10))
 (segment (start 127 91.44) (end 142.24 106.68) (width 0.8) (layer B.Cu) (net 26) (status 20))
 (segment (start 111.76 147.32) (end 111.76 149.86) (width 0.8) (layer B.Cu) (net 7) (status 20))
 (segment (start 101.6 137.16) (end 111.76 147.32) (width 0.8) (layer B.Cu) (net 7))
 (segment (start 101.6 109.22) (end 101.6 137.16) (width 0.8) (layer B.Cu) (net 7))
 (segment (start 83.82 101.6) (end 93.98 101.6) (width 0.8) (layer B.Cu) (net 7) (status 10))
 (segment (start 93.98 101.6) (end 101.6 109.22) (width 0.8) (layer B.Cu) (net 7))
 (segment (start 88.9 152.4) (end 88.9 149.86) (width 0.8) (layer B.Cu) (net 7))
 (segment (start 91.44 154.94) (end 88.9 152.4) (width 0.8) (layer B.Cu) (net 7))
 (segment (start 96.52 152.4) (end 93.98 154.94) (width 0.8) (layer B.Cu) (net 7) (status 10))
 (segment (start 93.98 154.94) (end 91.44 154.94) (width 0.8) (layer B.Cu) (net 7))
 (segment (start 81.28 151.13) (end 82.55 149.86) (width 0.8) (layer B.Cu) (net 7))
 (segment (start 81.28 152.4) (end 81.28 151.13) (width 0.8) (layer B.Cu) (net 7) (status 10))
 (segment (start 82.55 149.86) (end 88.9 149.86) (width 0.8) (layer B.Cu) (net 7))
 (segment (start 95.25 113.03) (end 83.82 101.6) (width 0.8) (layer B.Cu) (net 7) (status 20))
 (segment (start 95.25 148.59) (end 95.25 113.03) (width 0.8) (layer B.Cu) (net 7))
 (segment (start 88.9 149.86) (end 93.98 149.86) (width 0.8) (layer B.Cu) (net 7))
 (segment (start 93.98 149.86) (end 95.25 148.59) (width 0.8) (layer B.Cu) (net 7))
 (segment (start 76.2 88.9) (end 73.66 88.9) (width 0.8) (layer B.Cu) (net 11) (status 20))
 (segment (start 81.28 93.98) (end 76.2 88.9) (width 0.8) (layer B.Cu) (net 11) (status 10))
 (segment (start 67.31 95.25) (end 73.66 88.9) (width 0.8) (layer B.Cu) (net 11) (status 20))
 (segment (start 63.5 95.25) (end 67.31 95.25) (width 0.8) (layer B.Cu) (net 11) (status 10))
 (segment (start 78.74 93.98) (end 81.28 96.52) (width 0.8) (layer B.Cu) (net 13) (status 20))
 (segment (start 73.66 93.98) (end 78.74 93.98) (width 0.8) (layer B.Cu) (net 13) (status 10))
 (segment (start 142.24 132.08) (end 144.78 132.08) (width 0.8) (layer B.Cu) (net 13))
 (segment (start 127 149.86) (end 127 147.32) (width 0.8) (layer B.Cu) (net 13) (status 10))
 (segment (start 127 147.32) (end 142.24 132.08) (width 0.8) (layer B.Cu) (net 13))
 (segment (start 53.34 101.6) (end 68.58 101.6) (width 0.8) (layer B.Cu) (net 13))
 (segment (start 73.66 93.98) (end 71.12 96.52) (width 0.8) (layer B.Cu) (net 13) (status 10))
 (segment (start 71.12 96.52) (end 71.12 99.06) (width 0.8) (layer B.Cu) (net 13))
 (segment (start 71.12 99.06) (end 68.58 101.6) (width 0.8) (layer B.Cu) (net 13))
 (segment (start 134.62 157.48) (end 144.78 147.32) (width 0.8) (layer B.Cu) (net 13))
 (segment (start 144.78 104.14) (end 142.24 101.6) (width 0.8) (layer B.Cu) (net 13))
 (segment (start 144.78 147.32) (end 144.78 104.14) (width 0.8) (layer B.Cu) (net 13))
 (segment (start 63.5 89.25) (end 55.53 89.25) (width 0.8) (layer B.Cu) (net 13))
 (segment (start 55.53 89.25) (end 53.34 91.44) (width 0.8) (layer B.Cu) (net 13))
 (segment (start 53.34 91.44) (end 53.34 144.78) (width 0.8) (layer B.Cu) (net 13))
 (segment (start 53.34 144.78) (end 50.8 147.32) (width 0.8) (layer B.Cu) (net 13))
 (segment (start 50.8 149.86) (end 58.42 157.48) (width 0.8) (layer B.Cu) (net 13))
 (segment (start 50.8 147.32) (end 50.8 149.86) (width 0.8) (layer B.Cu) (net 13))
 (segment (start 127 154.94) (end 127 157.48) (width 0.8) (layer B.Cu) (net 13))
 (segment (start 58.42 157.48) (end 127 157.48) (width 0.8) (layer B.Cu) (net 13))
 (segment (start 127 157.48) (end 134.62 157.48) (width 0.8) (layer B.Cu) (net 13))
 (segment (start 96.52 91.44) (end 83.82 91.44) (width 0.8) (layer B.Cu) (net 8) (status 20))
 (segment (start 105.41 100.33) (end 96.52 91.44) (width 0.8) (layer B.Cu) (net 8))
 (segment (start 109.22 156.21) (end 115.57 156.21) (width 0.8) (layer B.Cu) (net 8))
 (segment (start 109.22 149.86) (end 109.22 156.21) (width 0.8) (layer B.Cu) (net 8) (status 10))
 (segment (start 115.57 156.21) (end 119.38 152.4) (width 0.8) (layer B.Cu) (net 8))
 (segment (start 119.38 152.4) (end 119.38 147.32) (width 0.8) (layer B.Cu) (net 8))
 (segment (start 119.38 147.32) (end 105.41 133.08001) (width 0.8) (layer B.Cu) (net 8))
 (segment (start 105.41 133.08001) (end 105.41 100.33) (width 0.8) (layer B.Cu) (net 8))
 (segment (start 99.06 127) (end 99.06 152.4) (width 0.8) (layer B.Cu) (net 8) (status 30))
 (segment (start 99.06 156.21) (end 59.69 156.21) (width 0.8) (layer B.Cu) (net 8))
 (segment (start 99.06 156.21) (end 99.06 152.4) (width 0.8) (layer B.Cu) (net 8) (status 20))
 (segment (start 109.22 156.21) (end 99.06 156.21) (width 0.8) (layer B.Cu) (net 8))
 (segment (start 83.82 152.4) (end 83.82 156.21) (width 0.8) (layer B.Cu) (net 8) (status 10))
 (segment (start 59.69 156.21) (end 53.34 149.86) (width 0.8) (layer B.Cu) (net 8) (status 20))
 (segment (start 132.08 152.4) (end 127 152.4) (width 0.8) (layer B.Cu) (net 12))
 (segment (start 92.71 85.09) (end 80.01 85.09) (width 0.8) (layer B.Cu) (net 12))
 (segment (start 106.68 99.06) (end 92.71 85.09) (width 0.8) (layer B.Cu) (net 12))
 (segment (start 127 152.4) (end 106.68 132.08) (width 0.8) (layer B.Cu) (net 12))
 (segment (start 106.68 132.08) (end 106.68 99.06) (width 0.8) (layer B.Cu) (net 12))
 (segment (start 142.24 129.54) (end 123.19 148.59) (width 0.8) (layer B.Cu) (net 12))
 (segment (start 78.74 86.36) (end 80.01 85.09) (width 0.8) (layer B.Cu) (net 12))
 (segment (start 81.28 91.44) (end 78.74 88.9) (width 0.8) (layer B.Cu) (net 12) (status 10))
 (segment (start 78.74 88.9) (end 78.74 86.36) (width 0.8) (layer B.Cu) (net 12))
 (segment (start 142.24 129.54) (end 142.24 124.46) (width 0.8) (layer B.Cu) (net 12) (status 20))
 (segment (start 132.08 152.4) (end 134.62 149.86) (width 0.8) (layer B.Cu) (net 12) (status 20))
 (segment (start 132.08 152.4) (end 132.08 154.94) (width 0.8) (layer B.Cu) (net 12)))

